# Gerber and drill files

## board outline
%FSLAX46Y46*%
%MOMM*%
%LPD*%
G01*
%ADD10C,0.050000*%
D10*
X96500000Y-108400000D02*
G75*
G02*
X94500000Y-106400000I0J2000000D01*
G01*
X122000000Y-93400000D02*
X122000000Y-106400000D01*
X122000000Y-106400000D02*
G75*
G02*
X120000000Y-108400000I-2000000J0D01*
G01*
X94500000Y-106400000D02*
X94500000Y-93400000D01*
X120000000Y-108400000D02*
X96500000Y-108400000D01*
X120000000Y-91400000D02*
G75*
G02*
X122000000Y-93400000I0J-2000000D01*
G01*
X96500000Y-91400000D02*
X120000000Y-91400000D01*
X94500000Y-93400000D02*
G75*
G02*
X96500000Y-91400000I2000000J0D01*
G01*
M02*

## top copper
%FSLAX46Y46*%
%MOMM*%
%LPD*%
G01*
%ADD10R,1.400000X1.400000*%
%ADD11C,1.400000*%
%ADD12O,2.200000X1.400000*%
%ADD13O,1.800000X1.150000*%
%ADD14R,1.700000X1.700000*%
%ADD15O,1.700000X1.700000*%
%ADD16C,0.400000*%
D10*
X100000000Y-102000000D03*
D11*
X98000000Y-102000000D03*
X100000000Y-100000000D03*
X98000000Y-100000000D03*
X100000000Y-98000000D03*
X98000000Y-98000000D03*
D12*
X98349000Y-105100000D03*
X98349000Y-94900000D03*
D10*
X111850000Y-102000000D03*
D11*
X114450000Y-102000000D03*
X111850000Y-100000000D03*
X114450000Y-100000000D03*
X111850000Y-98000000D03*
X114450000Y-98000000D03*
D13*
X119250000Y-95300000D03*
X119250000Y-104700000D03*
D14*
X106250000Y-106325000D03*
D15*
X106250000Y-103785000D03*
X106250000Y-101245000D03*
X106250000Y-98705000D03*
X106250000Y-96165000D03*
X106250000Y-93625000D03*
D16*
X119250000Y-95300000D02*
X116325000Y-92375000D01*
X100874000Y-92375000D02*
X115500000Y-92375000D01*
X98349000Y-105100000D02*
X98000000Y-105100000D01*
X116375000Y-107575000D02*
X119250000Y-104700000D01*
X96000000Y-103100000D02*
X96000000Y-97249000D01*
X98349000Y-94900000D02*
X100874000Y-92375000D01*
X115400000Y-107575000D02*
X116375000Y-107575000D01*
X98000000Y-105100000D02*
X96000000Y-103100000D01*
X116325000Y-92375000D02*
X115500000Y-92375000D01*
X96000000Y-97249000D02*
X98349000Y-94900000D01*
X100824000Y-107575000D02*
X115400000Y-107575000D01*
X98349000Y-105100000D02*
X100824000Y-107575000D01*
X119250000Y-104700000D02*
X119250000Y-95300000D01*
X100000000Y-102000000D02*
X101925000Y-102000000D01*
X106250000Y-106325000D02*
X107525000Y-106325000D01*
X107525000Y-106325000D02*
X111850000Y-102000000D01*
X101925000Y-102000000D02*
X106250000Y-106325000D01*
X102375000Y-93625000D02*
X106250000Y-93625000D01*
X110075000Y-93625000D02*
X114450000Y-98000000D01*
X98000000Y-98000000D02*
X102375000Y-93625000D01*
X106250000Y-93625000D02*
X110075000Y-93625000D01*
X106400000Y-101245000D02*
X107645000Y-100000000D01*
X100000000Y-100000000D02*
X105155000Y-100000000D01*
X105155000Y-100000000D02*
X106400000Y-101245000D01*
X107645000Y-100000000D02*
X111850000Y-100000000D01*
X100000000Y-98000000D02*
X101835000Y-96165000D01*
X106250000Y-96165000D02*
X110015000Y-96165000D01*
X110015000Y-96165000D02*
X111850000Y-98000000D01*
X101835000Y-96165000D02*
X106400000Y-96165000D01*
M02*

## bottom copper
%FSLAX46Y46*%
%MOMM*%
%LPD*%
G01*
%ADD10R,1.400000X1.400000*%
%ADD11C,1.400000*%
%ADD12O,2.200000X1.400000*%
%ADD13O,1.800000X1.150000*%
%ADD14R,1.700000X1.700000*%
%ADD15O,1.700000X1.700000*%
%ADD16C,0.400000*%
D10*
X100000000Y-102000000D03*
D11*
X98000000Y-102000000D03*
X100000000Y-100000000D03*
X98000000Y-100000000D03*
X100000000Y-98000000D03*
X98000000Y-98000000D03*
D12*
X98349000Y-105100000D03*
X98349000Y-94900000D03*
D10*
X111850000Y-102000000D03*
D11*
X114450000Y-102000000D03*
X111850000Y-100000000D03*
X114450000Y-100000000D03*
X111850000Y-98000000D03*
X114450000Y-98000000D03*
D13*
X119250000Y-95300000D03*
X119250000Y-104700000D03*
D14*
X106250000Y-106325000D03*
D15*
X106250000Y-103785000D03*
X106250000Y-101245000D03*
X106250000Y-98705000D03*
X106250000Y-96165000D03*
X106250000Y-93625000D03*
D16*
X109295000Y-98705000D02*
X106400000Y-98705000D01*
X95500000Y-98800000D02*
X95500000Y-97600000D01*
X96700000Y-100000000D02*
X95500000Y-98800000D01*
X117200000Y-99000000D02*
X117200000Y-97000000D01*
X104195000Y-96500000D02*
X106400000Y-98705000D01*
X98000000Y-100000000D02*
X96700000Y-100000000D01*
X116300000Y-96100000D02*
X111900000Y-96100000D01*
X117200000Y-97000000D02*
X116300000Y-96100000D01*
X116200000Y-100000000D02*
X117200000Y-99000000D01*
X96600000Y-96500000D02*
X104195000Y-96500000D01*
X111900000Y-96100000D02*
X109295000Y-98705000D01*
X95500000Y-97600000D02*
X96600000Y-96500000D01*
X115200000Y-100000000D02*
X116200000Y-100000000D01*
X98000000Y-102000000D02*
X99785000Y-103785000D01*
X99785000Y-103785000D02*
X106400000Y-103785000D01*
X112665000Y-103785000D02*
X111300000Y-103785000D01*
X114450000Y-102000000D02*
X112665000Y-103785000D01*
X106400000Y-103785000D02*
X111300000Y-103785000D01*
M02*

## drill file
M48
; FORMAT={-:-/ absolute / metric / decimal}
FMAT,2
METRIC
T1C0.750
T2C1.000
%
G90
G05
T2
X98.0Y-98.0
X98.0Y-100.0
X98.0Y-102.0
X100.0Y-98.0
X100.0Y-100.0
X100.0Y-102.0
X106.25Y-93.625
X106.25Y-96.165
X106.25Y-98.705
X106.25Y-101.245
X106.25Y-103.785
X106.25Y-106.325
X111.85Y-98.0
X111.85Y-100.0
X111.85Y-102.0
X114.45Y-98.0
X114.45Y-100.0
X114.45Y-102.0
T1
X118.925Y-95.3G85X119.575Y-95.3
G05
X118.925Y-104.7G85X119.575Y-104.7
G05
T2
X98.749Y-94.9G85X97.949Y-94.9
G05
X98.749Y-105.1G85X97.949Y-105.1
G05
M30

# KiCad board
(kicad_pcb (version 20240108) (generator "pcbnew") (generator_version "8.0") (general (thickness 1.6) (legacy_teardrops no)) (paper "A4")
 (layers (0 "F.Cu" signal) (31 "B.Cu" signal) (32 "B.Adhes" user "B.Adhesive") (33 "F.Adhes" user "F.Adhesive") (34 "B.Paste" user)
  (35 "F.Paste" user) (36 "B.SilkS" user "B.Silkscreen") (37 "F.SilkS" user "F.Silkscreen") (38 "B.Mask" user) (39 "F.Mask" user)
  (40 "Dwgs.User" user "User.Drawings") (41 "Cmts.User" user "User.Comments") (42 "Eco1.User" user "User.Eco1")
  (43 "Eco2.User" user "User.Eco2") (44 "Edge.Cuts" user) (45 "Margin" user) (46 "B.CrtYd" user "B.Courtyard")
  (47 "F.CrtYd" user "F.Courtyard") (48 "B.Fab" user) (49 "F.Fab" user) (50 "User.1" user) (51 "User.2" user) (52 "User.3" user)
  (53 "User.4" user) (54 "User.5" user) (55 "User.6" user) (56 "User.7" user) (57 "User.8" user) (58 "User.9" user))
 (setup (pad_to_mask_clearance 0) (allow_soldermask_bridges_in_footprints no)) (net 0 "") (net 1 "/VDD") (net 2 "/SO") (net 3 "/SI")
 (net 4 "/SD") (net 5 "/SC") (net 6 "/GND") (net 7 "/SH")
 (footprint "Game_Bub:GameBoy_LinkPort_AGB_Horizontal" (layer "F.Cu") (at 100 102 180)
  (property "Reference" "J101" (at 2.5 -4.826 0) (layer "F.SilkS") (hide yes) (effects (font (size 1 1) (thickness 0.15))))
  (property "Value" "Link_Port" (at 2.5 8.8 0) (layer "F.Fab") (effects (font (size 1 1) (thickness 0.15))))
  (pad "1" thru_hole rect (at 0 0 180) (size 1.4 1.4) (drill 1) (layers "*.Cu" "*.Mask") (remove_unused_layers no) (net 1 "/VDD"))
  (pad "2" thru_hole circle (at 2 0 180) (size 1.4 1.4) (drill 1) (layers "*.Cu" "*.Mask") (remove_unused_layers no) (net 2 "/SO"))
  (pad "3" thru_hole circle (at 0 2 180) (size 1.4 1.4) (drill 1) (layers "*.Cu" "*.Mask") (remove_unused_layers no) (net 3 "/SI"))
  (pad "4" thru_hole circle (at 2 2 180) (size 1.4 1.4) (drill 1) (layers "*.Cu" "*.Mask") (remove_unused_layers no) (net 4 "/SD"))
  (pad "5" thru_hole circle (at 0 4 180) (size 1.4 1.4) (drill 1) (layers "*.Cu" "*.Mask") (remove_unused_layers no) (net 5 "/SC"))
  (pad "6" thru_hole circle (at 2 4 180) (size 1.4 1.4) (drill 1) (layers "*.Cu" "*.Mask") (remove_unused_layers no) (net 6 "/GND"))
  (pad "SH" thru_hole oval (at 1.651 -3.1 270) (size 1.4 2.2) (drill oval 1 1.8) (layers "*.Cu" "*.Mask") (remove_unused_layers no)
   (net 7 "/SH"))
  (pad "SH" thru_hole oval (at 1.651 7.1 270) (size 1.4 2.2) (drill oval 1 1.8) (layers "*.Cu" "*.Mask") (remove_unused_layers no)
   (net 7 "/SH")))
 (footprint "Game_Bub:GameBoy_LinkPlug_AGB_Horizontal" (layer "F.Cu") (at 119.25 100)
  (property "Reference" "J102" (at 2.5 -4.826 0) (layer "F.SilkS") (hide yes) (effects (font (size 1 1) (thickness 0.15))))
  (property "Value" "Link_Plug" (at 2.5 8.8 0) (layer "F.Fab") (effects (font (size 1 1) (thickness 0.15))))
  (pad "1" thru_hole rect (at -7.4 2) (size 1.4 1.4) (drill 1) (layers "*.Cu" "*.Mask") (remove_unused_layers no) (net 1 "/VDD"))
  (pad "2" thru_hole circle (at -4.8 2) (size 1.4 1.4) (drill 1) (layers "*.Cu" "*.Mask") (remove_unused_layers no) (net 2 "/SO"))
  (pad "3" thru_hole circle (at -7.4 0) (size 1.4 1.4) (drill 1) (layers "*.Cu" "*.Mask") (remove_unused_layers no) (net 3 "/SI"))
  (pad "4" thru_hole circle (at -4.8 0) (size 1.4 1.4) (drill 1) (layers "*.Cu" "*.Mask") (remove_unused_layers no) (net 4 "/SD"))
  (pad "5" thru_hole circle (at -7.4 -2) (size 1.4 1.4) (drill 1) (layers "*.Cu" "*.Mask") (remove_unused_layers no) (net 5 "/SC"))
  (pad "6" thru_hole circle (at -4.8 -2) (size 1.4 1.4) (drill 1) (layers "*.Cu" "*.Mask") (remove_unused_layers no) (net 6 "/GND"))
  (pad "SH" thru_hole oval (at 0 -4.7 90) (size 1.15 1.8) (drill oval 0.75 1.4) (layers "*.Cu" "*.Mask") (remove_unused_layers no)
   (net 7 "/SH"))
  (pad "SH" thru_hole oval (at 0 4.7 90) (size 1.15 1.8) (drill oval 0.75 1.4) (layers "*.Cu" "*.Mask") (remove_unused_layers no)
   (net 7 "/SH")))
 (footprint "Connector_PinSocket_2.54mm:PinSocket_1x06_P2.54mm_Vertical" (layer "F.Cu") (at 106.25 106.325 180)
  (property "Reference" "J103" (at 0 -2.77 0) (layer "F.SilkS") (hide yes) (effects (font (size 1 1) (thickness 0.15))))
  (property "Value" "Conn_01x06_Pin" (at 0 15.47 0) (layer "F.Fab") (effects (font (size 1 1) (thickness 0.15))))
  (pad "1" thru_hole rect (at 0 0 180) (size 1.7 1.7) (drill 1) (layers "*.Cu" "*.Mask") (remove_unused_layers no) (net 1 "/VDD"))
  (pad "2" thru_hole oval (at 0 2.54 180) (size 1.7 1.7) (drill 1) (layers "*.Cu" "*.Mask") (remove_unused_layers no) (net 2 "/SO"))
  (pad "3" thru_hole oval (at 0 5.08 180) (size 1.7 1.7) (drill 1) (layers "*.Cu" "*.Mask") (remove_unused_layers no) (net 3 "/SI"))
  (pad "4" thru_hole oval (at 0 7.62 180) (size 1.7 1.7) (drill 1) (layers "*.Cu" "*.Mask") (remove_unused_layers no) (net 4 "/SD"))
  (pad "5" thru_hole oval (at 0 10.16 180) (size 1.7 1.7) (drill 1) (layers "*.Cu" "*.Mask") (remove_unused_layers no) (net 5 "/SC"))
  (pad "6" thru_hole oval (at 0 12.7 180) (size 1.7 1.7) (drill 1) (layers "*.Cu" "*.Mask") (remove_unused_layers no) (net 6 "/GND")))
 (gr_arc (start 96.5 108.4) (mid 95.085786 107.814214) (end 94.5 106.4) (stroke (width 0.05) (type default)) (layer "Edge.Cuts"))
 (gr_line (start 122 93.4) (end 122 106.4) (stroke (width 0.05) (type default)) (layer "Edge.Cuts"))
 (gr_arc (start 122 106.4) (mid 121.414214 107.814214) (end 120 108.4) (stroke (width 0.05) (type default)) (layer "Edge.Cuts"))
 (gr_line (start 94.5 106.4) (end 94.5 93.4) (stroke (width 0.05) (type default)) (layer "Edge.Cuts"))
 (gr_line (start 120 108.4) (end 96.5 108.4) (stroke (width 0.05) (type default)) (layer "Edge.Cuts"))
 (gr_arc (start 120 91.4) (mid 121.414214 91.985786) (end 122 93.4) (stroke (width 0.05) (type default)) (layer "Edge.Cuts"))
 (gr_line (start 96.5 91.4) (end 120 91.4) (stroke (width 0.05) (type default)) (layer "Edge.Cuts"))
 (gr_arc (start 94.5 93.4) (mid 95.085786 91.985786) (end 96.5 91.4) (stroke (width 0.05) (type default)) (layer "Edge.Cuts"))
 (segment (start 119.25 95.3) (end 116.325 92.375) (width 0.4) (layer "F.Cu") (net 7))
 (segment (start 100.874 92.375) (end 115.5 92.375) (width 0.4) (layer "F.Cu") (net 7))
 (segment (start 98.349 105.1) (end 98 105.1) (width 0.4) (layer "F.Cu") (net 7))
 (segment (start 116.375 107.575) (end 119.25 104.7) (width 0.4) (layer "F.Cu") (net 7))
 (segment (start 96 103.1) (end 96 97.249) (width 0.4) (layer "F.Cu") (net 7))
 (segment (start 98.349 94.9) (end 100.874 92.375) (width 0.4) (layer "F.Cu") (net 7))
 (segment (start 115.4 107.575) (end 116.375 107.575) (width 0.4) (layer "F.Cu") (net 7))
 (segment (start 98 105.1) (end 96 103.1) (width 0.4) (layer "F.Cu") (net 7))
 (segment (start 116.325 92.375) (end 115.5 92.375) (width 0.4) (layer "F.Cu") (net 7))
 (segment (start 96 97.249) (end 98.349 94.9) (width 0.4) (layer "F.Cu") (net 7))
 (segment (start 100.824 107.575) (end 115.4 107.575) (width 0.4) (layer "F.Cu") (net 7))
 (segment (start 98.349 105.1) (end 100.824 107.575) (width 0.4) (layer "F.Cu") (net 7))
 (segment (start 119.25 104.7) (end 119.25 95.3) (width 0.4) (layer "F.Cu") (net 7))
 (segment (start 100 102) (end 101.925 102) (width 0.4) (layer "F.Cu") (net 1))
 (segment (start 106.25 106.325) (end 107.525 106.325) (width 0.4) (layer "F.Cu") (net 1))
 (segment (start 107.525 106.325) (end 111.85 102) (width 0.4) (layer "F.Cu") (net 1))
 (segment (start 101.925 102) (end 106.25 106.325) (width 0.4) (layer "F.Cu") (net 1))
 (segment (start 109.295 98.705) (end 106.4 98.705) (width 0.4) (layer "B.Cu") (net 4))
 (segment (start 95.5 98.8) (end 95.5 97.6) (width 0.4) (layer "B.Cu") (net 4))
 (segment (start 96.7 100) (end 95.5 98.8) (width 0.4) (layer "B.Cu") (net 4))
 (segment (start 117.2 99) (end 117.2 97) (width 0.4) (layer "B.Cu") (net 4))
 (segment (start 104.195 96.5) (end 106.4 98.705) (width 0.4) (layer "B.Cu") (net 4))
 (segment (start 98 100) (end 96.7 100) (width 0.4) (layer "B.Cu") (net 4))
 (segment (start 116.3 96.1) (end 111.9 96.1) (width 0.4) (layer "B.Cu") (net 4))
 (segment (start 117.2 97) (end 116.3 96.1) (width 0.4) (layer "B.Cu") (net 4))
 (segment (start 116.2 100) (end 117.2 99) (width 0.4) (layer "B.Cu") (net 4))
 (segment (start 96.6 96.5) (end 104.195 96.5) (width 0.4) (layer "B.Cu") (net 4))
 (segment (start 111.9 96.1) (end 109.295 98.705) (width 0.4) (layer "B.Cu") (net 4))
 (segment (start 95.5 97.6) (end 96.6 96.5) (width 0.4) (layer "B.Cu") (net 4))
 (segment (start 115.2 100) (end 116.2 100) (width 0.4) (layer "B.Cu") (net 4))
 (segment (start 102.375 93.625) (end 106.25 93.625) (width 0.4) (layer "F.Cu") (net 6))
 (segment (start 110.075 93.625) (end 114.45 98) (width 0.4) (layer "F.Cu") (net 6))
 (segment (start 98 98) (end 102.375 93.625) (width 0.4) (layer "F.Cu") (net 6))
 (segment (start 106.25 93.625) (end 110.075 93.625) (width 0.4) (layer "F.Cu") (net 6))
 (segment (start 106.4 101.245) (end 107.645 100) (width 0.4) (layer "F.Cu") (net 3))
 (segment (start 100 100) (end 105.155 100) (width 0.4) (layer "F.Cu") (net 3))
 (segment (start 105.155 100) (end 106.4 101.245) (width 0.4) (layer "F.Cu") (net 3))
 (segment (start 107.645 100) (end 111.85 100) (width 0.4) (layer "F.Cu") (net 3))
 (segment (start 100 98) (end 101.835 96.165) (width 0.4) (layer "F.Cu") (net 5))
 (segment (start 106.25 96.165) (end 110.015 96.165) (width 0.4) (layer "F.Cu") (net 5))
 (segment (start 110.015 96.165) (end 111.85 98) (width 0.4) (layer "F.Cu") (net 5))
 (segment (start 101.835 96.165) (end 106.4 96.165) (width 0.4) (layer "F.Cu") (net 5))
 (segment (start 98 102) (end 99.785 103.785) (width 0.4) (layer "B.Cu") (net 2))
 (segment (start 99.785 103.785) (end 106.4 103.785) (width 0.4) (layer "B.Cu") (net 2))
 (segment (start 112.665 103.785) (end 111.3 103.785) (width 0.4) (layer "B.Cu") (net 2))
 (segment (start 114.45 102) (end 112.665 103.785) (width 0.4) (layer "B.Cu") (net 2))
 (segment (start 106.4 103.785) (end 111.3 103.785) (width 0.4) (layer "B.Cu") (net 2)))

